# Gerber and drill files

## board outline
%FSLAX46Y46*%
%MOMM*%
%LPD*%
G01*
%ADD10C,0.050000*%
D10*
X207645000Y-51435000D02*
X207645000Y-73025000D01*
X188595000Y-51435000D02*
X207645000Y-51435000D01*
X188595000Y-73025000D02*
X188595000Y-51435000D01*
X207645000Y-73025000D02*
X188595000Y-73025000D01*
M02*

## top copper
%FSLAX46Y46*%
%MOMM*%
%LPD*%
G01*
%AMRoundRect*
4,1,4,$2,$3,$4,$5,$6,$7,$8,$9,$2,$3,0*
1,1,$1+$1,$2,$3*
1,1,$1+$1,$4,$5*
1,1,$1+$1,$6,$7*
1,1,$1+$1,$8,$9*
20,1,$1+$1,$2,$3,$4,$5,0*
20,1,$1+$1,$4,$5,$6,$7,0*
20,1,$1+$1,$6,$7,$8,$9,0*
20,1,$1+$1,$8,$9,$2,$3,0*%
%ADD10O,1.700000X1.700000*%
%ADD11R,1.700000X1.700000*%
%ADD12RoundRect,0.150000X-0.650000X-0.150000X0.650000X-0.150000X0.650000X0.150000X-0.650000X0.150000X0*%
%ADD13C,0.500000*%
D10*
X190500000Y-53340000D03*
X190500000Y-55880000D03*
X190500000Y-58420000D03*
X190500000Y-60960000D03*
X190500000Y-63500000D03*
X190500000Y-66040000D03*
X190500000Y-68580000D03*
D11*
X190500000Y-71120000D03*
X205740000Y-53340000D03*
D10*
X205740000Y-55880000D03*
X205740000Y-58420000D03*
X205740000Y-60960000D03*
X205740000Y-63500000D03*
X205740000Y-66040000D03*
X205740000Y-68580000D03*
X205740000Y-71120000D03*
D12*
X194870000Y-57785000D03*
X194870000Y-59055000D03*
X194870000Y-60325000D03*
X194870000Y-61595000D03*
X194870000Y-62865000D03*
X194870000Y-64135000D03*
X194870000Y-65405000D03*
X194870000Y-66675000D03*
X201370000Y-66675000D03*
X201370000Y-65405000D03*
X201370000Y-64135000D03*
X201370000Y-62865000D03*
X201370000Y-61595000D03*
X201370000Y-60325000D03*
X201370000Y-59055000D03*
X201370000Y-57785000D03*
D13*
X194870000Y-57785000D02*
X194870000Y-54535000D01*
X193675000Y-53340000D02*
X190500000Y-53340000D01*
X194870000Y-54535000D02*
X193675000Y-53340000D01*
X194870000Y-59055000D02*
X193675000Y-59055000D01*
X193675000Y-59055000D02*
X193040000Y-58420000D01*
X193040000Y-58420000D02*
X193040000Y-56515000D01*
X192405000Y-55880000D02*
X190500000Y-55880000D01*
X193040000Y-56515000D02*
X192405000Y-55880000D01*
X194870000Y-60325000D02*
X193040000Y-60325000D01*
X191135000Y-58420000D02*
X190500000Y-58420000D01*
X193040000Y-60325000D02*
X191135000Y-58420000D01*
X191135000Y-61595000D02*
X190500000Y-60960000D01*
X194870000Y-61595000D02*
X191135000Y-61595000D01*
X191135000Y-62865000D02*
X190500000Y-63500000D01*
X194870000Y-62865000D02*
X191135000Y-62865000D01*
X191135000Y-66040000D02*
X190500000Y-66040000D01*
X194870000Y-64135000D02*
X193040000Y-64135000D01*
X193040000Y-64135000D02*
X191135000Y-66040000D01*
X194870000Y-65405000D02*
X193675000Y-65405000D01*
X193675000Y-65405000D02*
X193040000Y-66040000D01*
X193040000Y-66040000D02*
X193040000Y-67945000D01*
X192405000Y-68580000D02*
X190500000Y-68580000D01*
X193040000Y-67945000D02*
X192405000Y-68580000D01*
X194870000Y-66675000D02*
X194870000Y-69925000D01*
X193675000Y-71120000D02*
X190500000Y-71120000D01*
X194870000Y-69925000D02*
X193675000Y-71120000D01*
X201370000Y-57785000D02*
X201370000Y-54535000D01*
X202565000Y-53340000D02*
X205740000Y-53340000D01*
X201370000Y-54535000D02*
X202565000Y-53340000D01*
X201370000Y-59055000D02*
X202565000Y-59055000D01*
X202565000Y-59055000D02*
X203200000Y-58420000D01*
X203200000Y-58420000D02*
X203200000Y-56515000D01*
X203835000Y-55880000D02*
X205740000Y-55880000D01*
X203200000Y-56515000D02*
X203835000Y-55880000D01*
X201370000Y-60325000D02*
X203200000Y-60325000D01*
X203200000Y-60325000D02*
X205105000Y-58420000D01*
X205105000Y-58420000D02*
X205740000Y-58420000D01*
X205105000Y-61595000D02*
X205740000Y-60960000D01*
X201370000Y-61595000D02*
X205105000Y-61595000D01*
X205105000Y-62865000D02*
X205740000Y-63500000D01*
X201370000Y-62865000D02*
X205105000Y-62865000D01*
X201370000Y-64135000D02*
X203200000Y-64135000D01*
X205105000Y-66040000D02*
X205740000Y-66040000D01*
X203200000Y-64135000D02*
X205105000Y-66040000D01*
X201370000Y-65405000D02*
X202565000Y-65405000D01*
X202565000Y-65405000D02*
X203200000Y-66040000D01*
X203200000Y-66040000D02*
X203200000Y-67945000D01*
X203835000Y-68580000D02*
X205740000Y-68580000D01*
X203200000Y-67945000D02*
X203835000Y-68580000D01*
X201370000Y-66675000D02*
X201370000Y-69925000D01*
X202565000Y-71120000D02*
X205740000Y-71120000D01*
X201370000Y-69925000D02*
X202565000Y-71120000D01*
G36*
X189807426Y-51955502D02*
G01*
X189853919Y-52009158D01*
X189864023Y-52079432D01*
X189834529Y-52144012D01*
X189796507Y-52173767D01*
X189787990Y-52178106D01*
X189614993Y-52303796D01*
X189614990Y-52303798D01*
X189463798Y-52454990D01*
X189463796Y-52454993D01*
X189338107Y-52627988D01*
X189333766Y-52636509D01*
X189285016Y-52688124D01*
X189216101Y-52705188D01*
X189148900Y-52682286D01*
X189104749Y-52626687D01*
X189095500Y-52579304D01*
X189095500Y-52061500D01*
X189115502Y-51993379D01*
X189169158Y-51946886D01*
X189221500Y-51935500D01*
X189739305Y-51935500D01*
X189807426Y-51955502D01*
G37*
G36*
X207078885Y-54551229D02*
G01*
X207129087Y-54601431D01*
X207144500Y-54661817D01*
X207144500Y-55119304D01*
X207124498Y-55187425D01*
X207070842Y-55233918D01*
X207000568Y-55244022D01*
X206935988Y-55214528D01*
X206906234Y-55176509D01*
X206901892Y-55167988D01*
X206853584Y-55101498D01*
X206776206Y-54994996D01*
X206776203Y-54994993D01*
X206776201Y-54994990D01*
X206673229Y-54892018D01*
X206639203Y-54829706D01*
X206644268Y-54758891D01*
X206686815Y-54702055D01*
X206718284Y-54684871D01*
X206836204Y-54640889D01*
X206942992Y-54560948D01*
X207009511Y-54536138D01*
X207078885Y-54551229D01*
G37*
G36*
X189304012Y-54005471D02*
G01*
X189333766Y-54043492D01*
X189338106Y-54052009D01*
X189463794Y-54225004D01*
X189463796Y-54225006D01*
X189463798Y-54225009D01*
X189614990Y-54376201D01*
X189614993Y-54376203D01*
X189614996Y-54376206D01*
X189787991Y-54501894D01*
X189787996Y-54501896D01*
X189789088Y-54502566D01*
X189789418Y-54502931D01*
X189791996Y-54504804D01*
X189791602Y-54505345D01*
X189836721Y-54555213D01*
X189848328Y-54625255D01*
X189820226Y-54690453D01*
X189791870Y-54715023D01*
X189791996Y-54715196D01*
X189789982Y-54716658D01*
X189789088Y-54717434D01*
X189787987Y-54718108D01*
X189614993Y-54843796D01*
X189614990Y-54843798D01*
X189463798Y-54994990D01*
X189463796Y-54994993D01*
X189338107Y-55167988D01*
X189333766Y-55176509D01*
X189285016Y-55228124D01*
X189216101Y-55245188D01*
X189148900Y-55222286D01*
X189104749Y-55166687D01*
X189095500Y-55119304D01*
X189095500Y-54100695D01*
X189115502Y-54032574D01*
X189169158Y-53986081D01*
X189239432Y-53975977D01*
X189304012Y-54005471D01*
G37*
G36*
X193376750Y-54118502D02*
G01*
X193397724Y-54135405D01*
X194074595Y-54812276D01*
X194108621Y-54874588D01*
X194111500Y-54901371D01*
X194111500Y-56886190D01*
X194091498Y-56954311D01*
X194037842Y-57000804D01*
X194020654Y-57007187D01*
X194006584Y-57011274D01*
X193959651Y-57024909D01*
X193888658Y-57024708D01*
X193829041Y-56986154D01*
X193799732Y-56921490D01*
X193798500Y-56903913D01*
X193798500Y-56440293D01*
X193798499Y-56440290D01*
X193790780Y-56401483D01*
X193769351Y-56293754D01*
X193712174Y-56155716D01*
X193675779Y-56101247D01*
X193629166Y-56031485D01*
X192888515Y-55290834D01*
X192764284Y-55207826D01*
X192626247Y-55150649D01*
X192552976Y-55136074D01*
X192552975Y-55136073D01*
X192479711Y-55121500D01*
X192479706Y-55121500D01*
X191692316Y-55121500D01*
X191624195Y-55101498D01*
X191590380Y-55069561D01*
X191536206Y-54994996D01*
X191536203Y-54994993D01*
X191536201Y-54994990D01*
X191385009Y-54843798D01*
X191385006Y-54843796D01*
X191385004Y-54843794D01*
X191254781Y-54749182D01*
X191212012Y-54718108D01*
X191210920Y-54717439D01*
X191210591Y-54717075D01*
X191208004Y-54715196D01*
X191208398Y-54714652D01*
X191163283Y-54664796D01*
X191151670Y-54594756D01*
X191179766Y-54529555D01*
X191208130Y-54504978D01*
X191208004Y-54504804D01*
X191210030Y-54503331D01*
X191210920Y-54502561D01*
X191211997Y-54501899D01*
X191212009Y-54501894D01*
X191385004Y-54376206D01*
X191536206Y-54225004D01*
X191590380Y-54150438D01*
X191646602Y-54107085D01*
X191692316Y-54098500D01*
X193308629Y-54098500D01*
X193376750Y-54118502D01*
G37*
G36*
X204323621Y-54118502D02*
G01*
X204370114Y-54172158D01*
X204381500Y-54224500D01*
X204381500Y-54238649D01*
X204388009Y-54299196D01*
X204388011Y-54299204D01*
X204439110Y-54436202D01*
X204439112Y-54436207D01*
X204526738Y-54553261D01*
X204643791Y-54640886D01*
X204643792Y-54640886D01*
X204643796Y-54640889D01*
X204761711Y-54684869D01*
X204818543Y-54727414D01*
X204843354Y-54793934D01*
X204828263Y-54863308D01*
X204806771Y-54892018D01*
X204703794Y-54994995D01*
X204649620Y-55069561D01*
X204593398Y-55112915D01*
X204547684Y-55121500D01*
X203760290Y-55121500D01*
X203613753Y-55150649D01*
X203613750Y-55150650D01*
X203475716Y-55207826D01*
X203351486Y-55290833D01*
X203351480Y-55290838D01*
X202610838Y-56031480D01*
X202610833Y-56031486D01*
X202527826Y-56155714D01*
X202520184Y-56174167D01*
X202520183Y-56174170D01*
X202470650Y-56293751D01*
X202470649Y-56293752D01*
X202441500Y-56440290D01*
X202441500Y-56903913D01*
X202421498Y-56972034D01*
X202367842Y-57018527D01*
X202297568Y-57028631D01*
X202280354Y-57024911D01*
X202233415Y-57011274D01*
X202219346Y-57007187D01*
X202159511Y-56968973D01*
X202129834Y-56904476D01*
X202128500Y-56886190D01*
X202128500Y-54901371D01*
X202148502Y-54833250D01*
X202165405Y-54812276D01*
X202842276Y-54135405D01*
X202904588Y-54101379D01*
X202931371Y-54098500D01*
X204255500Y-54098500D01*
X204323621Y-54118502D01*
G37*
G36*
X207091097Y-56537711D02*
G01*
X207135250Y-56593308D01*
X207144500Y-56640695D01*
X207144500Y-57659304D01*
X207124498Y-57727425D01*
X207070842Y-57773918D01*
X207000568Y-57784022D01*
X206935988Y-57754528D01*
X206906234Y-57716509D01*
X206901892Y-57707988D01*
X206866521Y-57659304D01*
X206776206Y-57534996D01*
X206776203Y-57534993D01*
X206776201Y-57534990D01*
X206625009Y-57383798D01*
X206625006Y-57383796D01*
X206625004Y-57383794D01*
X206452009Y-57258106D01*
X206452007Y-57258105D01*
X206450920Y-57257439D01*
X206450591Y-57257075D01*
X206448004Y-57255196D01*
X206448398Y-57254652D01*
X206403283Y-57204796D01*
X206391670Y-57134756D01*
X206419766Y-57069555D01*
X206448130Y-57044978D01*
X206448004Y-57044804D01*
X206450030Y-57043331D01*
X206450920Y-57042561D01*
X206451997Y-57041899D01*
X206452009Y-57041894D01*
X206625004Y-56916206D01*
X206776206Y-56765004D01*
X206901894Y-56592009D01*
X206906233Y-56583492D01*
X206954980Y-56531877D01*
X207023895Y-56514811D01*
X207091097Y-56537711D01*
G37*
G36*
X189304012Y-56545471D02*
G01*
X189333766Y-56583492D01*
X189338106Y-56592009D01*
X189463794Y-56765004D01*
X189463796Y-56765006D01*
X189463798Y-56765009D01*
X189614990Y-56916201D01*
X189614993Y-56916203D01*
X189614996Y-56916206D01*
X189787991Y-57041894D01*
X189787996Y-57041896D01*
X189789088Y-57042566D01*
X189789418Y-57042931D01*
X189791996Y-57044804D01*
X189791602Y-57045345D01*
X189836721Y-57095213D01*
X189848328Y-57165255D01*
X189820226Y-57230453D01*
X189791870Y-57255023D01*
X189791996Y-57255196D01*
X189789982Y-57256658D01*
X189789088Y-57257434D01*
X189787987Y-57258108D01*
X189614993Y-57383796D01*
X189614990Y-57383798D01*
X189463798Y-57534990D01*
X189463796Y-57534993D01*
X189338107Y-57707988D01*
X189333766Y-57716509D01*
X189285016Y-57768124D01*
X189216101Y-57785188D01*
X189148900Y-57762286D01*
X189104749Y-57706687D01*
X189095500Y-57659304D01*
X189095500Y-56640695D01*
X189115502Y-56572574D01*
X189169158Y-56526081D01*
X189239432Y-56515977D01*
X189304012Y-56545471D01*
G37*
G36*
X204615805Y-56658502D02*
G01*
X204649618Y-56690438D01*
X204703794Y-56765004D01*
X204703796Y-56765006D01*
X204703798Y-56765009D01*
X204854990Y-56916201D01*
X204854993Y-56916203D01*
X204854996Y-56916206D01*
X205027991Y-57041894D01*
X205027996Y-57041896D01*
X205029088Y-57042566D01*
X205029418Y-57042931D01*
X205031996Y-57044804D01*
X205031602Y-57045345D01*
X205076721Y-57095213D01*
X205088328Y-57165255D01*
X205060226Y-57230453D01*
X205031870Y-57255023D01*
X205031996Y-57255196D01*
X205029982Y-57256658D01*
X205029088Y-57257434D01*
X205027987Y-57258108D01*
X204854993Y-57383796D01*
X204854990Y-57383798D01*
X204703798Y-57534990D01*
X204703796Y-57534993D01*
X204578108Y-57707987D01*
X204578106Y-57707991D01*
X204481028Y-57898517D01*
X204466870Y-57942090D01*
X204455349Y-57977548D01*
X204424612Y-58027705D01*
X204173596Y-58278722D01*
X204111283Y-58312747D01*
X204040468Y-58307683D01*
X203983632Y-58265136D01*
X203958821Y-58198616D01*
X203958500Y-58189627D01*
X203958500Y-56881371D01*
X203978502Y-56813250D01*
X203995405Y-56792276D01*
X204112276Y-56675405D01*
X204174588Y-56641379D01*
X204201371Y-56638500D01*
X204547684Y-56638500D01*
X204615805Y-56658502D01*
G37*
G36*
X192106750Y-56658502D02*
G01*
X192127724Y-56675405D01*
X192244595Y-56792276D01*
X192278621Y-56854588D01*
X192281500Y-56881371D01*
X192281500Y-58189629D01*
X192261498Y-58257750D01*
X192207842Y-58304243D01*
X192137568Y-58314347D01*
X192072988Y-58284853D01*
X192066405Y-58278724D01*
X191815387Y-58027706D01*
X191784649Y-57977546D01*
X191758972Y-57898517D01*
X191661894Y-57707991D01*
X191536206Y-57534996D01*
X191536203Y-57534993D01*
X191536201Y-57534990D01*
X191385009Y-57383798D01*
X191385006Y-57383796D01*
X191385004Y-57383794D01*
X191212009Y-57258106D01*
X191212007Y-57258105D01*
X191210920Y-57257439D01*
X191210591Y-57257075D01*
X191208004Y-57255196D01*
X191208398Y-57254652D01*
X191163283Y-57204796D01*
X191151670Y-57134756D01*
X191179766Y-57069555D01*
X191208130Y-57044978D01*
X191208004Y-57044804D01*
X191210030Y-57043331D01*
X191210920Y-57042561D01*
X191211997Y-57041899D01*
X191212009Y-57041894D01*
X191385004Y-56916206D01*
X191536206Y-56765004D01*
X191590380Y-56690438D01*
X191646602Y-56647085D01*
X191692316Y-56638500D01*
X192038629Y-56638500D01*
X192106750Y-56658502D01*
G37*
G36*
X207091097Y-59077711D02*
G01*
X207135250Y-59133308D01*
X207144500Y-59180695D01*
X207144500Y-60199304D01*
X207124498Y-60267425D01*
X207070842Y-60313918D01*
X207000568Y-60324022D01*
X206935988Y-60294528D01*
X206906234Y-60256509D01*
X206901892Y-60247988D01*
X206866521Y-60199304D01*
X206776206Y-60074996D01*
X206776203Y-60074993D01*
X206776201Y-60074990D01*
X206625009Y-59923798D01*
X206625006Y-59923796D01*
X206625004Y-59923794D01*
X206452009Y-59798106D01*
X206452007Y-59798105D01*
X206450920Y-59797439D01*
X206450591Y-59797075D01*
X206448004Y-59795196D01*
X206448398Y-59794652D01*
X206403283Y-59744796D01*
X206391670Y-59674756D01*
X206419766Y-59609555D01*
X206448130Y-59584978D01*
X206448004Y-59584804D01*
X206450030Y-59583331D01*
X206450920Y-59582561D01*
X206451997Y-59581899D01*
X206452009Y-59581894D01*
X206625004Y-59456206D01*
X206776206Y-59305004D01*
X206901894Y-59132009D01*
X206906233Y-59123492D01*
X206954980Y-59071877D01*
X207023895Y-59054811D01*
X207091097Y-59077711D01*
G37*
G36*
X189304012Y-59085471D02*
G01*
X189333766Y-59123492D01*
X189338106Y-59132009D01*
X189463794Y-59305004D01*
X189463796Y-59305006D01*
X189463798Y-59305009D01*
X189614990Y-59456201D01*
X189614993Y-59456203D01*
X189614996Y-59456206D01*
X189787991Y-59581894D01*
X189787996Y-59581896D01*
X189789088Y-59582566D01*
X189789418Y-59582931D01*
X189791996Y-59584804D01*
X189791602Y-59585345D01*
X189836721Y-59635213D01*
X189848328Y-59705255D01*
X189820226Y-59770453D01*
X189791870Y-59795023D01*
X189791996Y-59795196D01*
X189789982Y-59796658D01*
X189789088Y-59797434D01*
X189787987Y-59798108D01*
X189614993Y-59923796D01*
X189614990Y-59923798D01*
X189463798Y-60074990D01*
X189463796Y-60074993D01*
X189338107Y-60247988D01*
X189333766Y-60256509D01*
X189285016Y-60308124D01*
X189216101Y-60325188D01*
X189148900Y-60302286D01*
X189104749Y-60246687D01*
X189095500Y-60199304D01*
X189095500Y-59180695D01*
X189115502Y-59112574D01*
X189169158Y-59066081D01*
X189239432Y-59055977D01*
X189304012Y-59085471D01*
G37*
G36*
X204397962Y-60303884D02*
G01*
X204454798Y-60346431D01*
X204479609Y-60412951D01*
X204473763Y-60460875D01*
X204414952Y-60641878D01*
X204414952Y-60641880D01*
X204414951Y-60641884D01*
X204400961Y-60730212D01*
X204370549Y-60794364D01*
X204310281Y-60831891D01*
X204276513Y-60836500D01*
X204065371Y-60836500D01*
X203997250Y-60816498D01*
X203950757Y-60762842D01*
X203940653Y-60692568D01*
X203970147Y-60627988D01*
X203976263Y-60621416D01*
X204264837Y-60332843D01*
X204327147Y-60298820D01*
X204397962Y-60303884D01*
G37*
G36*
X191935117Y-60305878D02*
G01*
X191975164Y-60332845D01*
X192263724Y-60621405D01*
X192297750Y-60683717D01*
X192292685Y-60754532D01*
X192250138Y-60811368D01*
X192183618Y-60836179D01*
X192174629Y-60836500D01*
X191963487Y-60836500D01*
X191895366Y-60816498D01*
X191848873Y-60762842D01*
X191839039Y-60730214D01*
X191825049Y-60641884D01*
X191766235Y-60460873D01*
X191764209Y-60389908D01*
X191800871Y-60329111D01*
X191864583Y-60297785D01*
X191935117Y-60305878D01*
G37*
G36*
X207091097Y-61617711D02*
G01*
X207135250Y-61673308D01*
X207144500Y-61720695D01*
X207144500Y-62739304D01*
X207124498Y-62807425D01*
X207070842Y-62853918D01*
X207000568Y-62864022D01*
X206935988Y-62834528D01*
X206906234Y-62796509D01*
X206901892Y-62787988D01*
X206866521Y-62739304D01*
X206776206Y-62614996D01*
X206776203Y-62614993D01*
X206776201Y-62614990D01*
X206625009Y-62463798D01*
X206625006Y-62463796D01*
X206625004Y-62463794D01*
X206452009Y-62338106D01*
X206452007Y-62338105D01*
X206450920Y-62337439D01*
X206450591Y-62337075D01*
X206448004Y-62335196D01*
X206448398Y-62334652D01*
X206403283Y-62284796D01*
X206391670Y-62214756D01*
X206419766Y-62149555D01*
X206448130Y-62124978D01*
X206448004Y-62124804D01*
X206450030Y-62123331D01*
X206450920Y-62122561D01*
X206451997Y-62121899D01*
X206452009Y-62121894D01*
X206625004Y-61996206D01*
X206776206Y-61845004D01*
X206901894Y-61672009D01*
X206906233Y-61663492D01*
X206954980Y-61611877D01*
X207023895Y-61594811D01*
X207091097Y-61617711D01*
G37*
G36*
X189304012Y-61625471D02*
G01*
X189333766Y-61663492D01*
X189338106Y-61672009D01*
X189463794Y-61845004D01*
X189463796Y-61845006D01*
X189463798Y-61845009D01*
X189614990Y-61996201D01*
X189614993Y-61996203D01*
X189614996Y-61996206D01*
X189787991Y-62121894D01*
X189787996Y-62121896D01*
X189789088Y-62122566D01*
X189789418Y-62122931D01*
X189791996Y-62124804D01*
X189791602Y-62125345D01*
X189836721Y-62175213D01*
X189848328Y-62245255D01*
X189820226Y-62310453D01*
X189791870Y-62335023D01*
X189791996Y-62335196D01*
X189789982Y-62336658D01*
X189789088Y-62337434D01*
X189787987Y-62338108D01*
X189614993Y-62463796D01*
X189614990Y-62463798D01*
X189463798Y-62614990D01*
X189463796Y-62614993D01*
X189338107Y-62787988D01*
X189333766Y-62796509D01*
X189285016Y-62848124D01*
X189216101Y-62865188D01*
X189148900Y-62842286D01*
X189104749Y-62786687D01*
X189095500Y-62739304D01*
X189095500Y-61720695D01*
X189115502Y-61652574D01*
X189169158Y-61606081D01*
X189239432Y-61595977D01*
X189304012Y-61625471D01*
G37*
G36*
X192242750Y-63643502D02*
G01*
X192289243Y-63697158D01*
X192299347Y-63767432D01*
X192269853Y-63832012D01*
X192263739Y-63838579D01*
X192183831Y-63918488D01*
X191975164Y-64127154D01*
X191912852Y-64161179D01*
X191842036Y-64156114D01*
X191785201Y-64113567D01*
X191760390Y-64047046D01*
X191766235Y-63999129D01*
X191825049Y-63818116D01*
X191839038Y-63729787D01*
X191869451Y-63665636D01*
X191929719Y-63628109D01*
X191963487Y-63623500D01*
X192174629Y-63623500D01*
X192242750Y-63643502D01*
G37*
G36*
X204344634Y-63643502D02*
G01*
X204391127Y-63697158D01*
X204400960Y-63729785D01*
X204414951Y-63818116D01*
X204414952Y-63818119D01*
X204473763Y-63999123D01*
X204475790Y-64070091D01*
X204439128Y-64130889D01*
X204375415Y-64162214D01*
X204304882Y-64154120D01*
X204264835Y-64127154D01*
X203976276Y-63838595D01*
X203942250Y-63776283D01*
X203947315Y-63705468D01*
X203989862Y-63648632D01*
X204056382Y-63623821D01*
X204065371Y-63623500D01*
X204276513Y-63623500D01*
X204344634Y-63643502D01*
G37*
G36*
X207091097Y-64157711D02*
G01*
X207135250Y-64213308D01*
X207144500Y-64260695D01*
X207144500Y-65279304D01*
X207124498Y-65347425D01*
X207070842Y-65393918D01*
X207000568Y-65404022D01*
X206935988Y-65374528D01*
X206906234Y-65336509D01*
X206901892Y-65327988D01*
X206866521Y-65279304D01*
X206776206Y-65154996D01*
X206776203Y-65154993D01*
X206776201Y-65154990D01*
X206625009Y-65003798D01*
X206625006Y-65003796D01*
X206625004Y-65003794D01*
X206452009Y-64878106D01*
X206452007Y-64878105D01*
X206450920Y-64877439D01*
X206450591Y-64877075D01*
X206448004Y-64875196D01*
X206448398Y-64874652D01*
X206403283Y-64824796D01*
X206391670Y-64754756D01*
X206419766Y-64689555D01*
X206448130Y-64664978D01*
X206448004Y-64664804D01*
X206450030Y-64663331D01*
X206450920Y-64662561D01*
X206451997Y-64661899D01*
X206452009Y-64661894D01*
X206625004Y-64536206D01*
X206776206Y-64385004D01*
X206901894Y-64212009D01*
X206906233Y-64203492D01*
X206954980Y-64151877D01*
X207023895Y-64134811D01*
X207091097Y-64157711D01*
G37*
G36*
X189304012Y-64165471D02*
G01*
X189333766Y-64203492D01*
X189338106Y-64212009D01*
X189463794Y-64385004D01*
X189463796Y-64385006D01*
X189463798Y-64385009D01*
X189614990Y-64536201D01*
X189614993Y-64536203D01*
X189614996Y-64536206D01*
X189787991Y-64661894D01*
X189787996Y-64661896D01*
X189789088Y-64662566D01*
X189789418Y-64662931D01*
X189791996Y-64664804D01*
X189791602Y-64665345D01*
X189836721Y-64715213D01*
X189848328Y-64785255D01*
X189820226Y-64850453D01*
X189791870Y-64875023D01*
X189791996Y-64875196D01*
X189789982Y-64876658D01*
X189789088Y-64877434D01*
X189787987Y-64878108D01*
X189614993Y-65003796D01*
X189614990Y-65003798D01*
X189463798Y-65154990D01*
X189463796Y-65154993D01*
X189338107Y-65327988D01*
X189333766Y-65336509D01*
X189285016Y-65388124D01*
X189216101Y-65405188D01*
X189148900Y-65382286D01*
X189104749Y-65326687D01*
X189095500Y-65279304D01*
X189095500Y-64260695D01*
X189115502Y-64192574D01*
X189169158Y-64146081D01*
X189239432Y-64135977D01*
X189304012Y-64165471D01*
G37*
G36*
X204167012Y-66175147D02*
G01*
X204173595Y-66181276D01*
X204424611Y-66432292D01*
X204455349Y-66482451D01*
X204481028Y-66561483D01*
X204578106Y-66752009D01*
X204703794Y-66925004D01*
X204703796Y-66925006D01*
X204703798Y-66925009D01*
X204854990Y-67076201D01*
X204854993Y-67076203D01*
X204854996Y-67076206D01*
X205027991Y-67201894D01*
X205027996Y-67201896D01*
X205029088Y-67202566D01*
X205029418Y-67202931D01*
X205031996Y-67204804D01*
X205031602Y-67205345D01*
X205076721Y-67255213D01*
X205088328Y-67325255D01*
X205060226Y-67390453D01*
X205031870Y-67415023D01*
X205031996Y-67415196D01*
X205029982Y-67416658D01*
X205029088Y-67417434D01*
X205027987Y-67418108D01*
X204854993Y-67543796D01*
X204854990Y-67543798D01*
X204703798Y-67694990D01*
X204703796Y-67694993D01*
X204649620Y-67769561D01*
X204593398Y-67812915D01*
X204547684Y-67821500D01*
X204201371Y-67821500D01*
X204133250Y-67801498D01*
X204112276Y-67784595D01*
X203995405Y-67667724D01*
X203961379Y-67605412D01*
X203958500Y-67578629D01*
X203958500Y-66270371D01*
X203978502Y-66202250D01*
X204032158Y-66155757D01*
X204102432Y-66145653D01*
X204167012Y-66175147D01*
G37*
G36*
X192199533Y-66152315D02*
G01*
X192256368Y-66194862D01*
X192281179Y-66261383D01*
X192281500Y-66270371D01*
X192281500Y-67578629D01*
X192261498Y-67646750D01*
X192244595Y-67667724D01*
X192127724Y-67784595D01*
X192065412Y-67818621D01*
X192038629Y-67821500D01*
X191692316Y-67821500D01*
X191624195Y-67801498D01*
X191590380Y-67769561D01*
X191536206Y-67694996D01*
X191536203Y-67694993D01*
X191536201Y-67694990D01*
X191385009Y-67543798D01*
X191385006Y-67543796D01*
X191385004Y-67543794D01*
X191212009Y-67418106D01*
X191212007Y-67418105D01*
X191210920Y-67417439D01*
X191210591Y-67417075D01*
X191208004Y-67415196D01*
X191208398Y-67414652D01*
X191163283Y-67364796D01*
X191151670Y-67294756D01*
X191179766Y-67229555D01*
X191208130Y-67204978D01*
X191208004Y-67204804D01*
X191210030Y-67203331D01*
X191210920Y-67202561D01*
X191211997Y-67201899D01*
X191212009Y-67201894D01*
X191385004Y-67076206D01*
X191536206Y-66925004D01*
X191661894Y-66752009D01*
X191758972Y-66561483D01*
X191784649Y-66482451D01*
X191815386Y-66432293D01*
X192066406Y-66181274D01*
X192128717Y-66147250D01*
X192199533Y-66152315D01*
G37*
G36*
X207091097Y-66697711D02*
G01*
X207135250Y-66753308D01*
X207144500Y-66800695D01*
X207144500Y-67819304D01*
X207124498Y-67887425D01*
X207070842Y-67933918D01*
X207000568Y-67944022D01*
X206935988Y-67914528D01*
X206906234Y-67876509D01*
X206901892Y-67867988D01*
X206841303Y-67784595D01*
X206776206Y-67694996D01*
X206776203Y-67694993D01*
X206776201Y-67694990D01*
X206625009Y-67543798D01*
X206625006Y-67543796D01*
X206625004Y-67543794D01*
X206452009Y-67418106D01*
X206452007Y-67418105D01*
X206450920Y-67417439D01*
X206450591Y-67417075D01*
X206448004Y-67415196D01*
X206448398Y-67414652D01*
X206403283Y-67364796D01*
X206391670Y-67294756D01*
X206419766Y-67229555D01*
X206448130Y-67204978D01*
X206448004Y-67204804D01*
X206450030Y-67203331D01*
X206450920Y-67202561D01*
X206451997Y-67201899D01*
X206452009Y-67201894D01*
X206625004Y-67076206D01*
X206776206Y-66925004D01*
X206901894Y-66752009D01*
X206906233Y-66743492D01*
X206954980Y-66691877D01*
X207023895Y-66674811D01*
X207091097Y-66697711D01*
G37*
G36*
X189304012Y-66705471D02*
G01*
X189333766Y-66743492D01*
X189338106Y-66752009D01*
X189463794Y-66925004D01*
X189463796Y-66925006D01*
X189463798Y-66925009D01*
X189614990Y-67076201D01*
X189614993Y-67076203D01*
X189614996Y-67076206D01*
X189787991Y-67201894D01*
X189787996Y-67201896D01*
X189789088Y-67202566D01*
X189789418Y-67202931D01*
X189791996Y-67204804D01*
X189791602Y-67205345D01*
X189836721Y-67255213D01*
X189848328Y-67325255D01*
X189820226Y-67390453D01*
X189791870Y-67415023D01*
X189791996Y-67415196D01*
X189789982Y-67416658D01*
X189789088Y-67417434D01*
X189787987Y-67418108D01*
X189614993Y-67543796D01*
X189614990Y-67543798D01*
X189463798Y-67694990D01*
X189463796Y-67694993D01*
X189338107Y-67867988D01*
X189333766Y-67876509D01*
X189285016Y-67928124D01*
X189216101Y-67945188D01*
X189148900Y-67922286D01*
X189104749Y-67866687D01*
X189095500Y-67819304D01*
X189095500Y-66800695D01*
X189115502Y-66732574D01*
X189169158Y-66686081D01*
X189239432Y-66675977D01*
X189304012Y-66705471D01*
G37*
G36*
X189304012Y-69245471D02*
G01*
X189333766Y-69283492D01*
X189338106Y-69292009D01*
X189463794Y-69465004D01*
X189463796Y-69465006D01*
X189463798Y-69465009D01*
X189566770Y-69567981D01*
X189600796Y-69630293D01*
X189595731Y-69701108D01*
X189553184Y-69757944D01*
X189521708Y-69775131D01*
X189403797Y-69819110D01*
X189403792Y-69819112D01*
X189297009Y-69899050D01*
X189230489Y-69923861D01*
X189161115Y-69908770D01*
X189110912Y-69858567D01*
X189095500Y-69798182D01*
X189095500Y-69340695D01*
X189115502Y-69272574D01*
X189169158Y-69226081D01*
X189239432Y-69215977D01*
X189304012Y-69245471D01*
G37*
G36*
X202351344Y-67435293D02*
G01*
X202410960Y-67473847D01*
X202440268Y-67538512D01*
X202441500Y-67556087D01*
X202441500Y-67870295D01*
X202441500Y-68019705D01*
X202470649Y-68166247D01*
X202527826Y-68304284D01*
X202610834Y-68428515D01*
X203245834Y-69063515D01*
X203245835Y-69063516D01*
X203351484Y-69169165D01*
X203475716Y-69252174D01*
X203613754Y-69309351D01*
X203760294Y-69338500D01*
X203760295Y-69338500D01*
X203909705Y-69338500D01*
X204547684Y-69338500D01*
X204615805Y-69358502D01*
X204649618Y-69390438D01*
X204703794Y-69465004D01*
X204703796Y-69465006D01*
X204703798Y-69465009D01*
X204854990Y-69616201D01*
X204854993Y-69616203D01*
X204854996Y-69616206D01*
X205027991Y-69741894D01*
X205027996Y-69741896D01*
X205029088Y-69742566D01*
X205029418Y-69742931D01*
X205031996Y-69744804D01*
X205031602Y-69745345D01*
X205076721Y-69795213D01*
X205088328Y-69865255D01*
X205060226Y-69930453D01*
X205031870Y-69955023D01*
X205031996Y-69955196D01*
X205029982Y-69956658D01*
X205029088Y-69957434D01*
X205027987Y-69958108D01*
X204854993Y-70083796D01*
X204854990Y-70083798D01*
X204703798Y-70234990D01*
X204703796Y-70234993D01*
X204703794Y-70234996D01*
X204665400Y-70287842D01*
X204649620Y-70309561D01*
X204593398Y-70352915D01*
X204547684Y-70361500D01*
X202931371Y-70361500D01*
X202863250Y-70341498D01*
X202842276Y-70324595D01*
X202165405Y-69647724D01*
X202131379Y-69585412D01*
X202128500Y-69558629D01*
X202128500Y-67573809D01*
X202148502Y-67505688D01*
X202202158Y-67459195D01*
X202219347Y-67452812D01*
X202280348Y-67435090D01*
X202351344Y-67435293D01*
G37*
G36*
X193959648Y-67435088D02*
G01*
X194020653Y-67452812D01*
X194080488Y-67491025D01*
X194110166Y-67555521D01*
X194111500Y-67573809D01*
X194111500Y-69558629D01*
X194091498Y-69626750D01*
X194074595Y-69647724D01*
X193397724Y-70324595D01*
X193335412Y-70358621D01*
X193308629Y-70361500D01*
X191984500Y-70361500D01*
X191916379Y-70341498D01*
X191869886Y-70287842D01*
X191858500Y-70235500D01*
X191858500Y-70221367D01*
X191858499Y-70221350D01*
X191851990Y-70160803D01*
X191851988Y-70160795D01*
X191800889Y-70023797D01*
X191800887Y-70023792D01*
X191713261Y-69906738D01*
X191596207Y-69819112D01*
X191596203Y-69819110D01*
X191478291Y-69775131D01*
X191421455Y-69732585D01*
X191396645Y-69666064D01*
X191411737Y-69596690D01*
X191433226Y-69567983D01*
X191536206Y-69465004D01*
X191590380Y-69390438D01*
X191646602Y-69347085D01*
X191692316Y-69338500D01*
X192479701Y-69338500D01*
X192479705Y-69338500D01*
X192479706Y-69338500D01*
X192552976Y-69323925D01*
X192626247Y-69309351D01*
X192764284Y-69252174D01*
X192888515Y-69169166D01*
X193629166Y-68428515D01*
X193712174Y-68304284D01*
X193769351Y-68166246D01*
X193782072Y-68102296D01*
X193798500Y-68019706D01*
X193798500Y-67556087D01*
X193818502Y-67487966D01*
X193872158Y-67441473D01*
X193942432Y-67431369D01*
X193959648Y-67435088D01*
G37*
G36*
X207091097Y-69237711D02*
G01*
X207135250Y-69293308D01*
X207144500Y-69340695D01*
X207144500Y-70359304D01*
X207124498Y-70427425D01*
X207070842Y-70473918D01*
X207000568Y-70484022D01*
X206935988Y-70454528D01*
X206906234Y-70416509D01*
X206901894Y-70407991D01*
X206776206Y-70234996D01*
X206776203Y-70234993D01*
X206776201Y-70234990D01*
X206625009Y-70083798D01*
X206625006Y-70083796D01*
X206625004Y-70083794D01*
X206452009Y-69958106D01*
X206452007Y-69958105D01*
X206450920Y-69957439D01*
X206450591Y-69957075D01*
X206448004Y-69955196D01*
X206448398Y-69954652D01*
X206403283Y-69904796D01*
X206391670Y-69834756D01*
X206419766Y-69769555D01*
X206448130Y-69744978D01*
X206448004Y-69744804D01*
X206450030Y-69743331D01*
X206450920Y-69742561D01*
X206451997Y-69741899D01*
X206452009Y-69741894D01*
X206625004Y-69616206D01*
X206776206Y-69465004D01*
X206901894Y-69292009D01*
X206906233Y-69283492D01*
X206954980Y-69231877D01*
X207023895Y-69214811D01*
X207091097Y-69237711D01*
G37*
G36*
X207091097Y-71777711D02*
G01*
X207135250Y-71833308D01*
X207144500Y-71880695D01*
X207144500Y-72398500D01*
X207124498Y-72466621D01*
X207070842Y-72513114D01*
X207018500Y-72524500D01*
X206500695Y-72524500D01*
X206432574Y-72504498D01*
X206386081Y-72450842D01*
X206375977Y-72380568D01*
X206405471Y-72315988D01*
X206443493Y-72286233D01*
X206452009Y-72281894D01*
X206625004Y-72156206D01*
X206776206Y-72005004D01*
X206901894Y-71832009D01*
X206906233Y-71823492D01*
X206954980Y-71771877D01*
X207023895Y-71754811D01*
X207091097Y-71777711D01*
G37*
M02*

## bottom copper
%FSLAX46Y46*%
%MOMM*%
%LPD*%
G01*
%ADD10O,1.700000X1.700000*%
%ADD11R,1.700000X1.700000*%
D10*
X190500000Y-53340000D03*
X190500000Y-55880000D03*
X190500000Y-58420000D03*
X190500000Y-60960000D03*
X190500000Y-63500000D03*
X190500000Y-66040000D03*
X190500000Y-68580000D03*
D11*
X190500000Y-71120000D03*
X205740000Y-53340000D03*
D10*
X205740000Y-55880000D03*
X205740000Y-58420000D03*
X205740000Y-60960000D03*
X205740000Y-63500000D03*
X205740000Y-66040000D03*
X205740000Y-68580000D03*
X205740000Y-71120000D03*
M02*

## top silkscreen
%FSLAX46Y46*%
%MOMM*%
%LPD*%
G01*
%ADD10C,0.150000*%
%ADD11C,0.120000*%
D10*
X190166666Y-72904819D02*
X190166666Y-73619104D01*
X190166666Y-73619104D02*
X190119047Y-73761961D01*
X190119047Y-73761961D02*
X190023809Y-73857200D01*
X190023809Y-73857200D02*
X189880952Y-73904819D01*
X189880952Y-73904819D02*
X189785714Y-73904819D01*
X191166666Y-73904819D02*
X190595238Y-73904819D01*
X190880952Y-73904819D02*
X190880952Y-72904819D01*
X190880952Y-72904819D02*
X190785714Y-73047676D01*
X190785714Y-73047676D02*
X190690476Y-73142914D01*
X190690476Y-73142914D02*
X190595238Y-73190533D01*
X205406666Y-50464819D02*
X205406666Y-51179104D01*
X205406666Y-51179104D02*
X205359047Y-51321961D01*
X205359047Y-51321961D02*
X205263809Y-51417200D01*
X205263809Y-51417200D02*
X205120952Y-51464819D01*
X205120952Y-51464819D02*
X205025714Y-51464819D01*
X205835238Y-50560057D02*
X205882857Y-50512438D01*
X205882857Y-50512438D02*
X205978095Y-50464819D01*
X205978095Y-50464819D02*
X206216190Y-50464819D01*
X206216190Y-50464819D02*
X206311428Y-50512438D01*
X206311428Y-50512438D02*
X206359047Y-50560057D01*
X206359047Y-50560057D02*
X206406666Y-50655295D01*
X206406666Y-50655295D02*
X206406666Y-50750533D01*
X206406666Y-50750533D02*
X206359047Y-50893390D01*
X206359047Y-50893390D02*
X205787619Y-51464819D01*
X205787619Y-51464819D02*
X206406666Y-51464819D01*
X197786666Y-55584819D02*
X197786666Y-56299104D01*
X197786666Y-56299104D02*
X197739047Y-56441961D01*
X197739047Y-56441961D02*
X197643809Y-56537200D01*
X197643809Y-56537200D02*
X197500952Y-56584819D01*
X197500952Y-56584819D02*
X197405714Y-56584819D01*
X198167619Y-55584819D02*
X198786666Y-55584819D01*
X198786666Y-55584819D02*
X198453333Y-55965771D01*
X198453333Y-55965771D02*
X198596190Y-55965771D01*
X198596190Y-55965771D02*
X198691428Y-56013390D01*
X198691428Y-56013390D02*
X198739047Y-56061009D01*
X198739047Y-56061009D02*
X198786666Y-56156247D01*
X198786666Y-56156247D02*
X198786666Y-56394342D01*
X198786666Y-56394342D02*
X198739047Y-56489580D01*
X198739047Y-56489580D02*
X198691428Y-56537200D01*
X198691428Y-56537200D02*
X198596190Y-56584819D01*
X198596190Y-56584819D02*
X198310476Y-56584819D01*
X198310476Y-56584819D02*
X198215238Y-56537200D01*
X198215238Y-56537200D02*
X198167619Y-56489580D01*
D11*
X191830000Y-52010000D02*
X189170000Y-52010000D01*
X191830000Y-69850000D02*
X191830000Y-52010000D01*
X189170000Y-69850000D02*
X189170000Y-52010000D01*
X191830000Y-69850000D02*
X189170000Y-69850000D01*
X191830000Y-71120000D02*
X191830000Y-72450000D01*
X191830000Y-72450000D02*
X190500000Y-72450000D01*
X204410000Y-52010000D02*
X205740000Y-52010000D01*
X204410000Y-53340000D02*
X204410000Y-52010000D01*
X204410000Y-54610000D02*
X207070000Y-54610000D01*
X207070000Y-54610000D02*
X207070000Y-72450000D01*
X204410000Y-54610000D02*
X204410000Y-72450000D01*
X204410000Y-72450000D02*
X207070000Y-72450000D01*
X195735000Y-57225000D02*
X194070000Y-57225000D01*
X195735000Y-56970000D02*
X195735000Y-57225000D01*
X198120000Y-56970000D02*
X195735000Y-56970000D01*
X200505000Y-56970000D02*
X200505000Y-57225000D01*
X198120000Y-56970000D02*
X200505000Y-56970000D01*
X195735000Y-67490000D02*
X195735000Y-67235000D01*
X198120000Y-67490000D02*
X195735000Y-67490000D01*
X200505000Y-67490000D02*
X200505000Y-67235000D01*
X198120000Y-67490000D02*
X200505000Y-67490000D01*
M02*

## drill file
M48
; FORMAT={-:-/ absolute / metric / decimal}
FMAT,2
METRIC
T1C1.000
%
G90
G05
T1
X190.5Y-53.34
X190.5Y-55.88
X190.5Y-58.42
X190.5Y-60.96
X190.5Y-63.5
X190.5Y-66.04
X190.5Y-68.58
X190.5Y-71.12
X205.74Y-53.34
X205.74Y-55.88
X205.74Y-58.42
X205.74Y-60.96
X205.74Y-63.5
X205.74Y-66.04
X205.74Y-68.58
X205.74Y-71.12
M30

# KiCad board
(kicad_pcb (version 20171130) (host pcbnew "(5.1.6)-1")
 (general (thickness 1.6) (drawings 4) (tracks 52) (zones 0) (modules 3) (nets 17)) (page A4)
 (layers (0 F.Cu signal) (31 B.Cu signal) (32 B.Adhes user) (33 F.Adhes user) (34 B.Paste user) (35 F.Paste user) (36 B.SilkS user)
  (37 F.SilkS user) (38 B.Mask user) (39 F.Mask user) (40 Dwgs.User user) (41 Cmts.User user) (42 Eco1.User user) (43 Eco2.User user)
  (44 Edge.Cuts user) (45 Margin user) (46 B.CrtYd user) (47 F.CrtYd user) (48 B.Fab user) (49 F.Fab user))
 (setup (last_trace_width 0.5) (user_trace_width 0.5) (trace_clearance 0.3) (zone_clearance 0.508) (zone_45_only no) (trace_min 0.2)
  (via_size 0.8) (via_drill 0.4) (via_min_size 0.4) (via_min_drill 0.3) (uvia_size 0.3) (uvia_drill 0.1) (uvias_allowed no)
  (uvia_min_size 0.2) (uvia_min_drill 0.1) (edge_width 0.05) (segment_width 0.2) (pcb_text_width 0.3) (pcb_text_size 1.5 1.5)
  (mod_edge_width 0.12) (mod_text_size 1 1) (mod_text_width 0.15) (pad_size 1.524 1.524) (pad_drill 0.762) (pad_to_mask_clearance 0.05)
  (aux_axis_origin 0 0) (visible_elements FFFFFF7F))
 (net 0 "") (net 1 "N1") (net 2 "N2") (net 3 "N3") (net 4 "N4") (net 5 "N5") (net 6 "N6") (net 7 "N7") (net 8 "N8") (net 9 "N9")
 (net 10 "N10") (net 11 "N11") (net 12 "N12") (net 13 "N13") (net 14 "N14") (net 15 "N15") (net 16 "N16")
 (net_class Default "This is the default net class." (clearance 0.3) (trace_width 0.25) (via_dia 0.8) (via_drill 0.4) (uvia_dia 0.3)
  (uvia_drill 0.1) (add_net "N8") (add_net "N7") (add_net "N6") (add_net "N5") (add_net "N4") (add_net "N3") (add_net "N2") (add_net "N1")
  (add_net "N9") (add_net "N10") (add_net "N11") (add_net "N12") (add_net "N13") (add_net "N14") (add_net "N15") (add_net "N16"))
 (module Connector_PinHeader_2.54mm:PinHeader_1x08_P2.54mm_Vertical (layer F.Cu) (at 190.5 71.12 180)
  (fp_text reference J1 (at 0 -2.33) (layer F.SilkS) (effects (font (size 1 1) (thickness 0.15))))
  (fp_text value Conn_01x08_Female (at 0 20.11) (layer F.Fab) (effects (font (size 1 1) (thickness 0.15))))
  (fp_line (start -1.33 19.11) (end 1.33 19.11) (layer F.SilkS) (width 0.12))
  (fp_line (start -1.33 1.27) (end -1.33 19.11) (layer F.SilkS) (width 0.12))
  (fp_line (start 1.33 1.27) (end 1.33 19.11) (layer F.SilkS) (width 0.12))
  (fp_line (start -1.33 1.27) (end 1.33 1.27) (layer F.SilkS) (width 0.12))
  (fp_line (start -1.33 0) (end -1.33 -1.33) (layer F.SilkS) (width 0.12))
  (fp_line (start -1.33 -1.33) (end 0 -1.33) (layer F.SilkS) (width 0.12))
  (pad 8 thru_hole oval (at 0 17.78 180) (size 1.7 1.7) (drill 1) (layers *.Cu *.Mask) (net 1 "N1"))
  (pad 7 thru_hole oval (at 0 15.24 180) (size 1.7 1.7) (drill 1) (layers *.Cu *.Mask) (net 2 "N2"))
  (pad 6 thru_hole oval (at 0 12.7 180) (size 1.7 1.7) (drill 1) (layers *.Cu *.Mask) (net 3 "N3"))
  (pad 5 thru_hole oval (at 0 10.16 180) (size 1.7 1.7) (drill 1) (layers *.Cu *.Mask) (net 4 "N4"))
  (pad 4 thru_hole oval (at 0 7.62 180) (size 1.7 1.7) (drill 1) (layers *.Cu *.Mask) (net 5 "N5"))
  (pad 3 thru_hole oval (at 0 5.08 180) (size 1.7 1.7) (drill 1) (layers *.Cu *.Mask) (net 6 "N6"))
  (pad 2 thru_hole oval (at 0 2.54 180) (size 1.7 1.7) (drill 1) (layers *.Cu *.Mask) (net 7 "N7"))
  (pad 1 thru_hole rect (at 0 0 180) (size 1.7 1.7) (drill 1) (layers *.Cu *.Mask) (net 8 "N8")))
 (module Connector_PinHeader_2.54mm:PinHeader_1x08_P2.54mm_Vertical (layer F.Cu) (at 205.74 53.34)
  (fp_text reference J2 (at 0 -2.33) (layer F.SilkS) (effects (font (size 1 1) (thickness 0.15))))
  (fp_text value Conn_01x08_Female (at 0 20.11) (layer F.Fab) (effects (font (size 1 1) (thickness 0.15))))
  (fp_line (start -1.33 -1.33) (end 0 -1.33) (layer F.SilkS) (width 0.12))
  (fp_line (start -1.33 0) (end -1.33 -1.33) (layer F.SilkS) (width 0.12))
  (fp_line (start -1.33 1.27) (end 1.33 1.27) (layer F.SilkS) (width 0.12))
  (fp_line (start 1.33 1.27) (end 1.33 19.11) (layer F.SilkS) (width 0.12))
  (fp_line (start -1.33 1.27) (end -1.33 19.11) (layer F.SilkS) (width 0.12))
  (fp_line (start -1.33 19.11) (end 1.33 19.11) (layer F.SilkS) (width 0.12))
  (pad 1 thru_hole rect (at 0 0) (size 1.7 1.7) (drill 1) (layers *.Cu *.Mask) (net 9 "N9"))
  (pad 2 thru_hole oval (at 0 2.54) (size 1.7 1.7) (drill 1) (layers *.Cu *.Mask) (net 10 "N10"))
  (pad 3 thru_hole oval (at 0 5.08) (size 1.7 1.7) (drill 1) (layers *.Cu *.Mask) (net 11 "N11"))
  (pad 4 thru_hole oval (at 0 7.62) (size 1.7 1.7) (drill 1) (layers *.Cu *.Mask) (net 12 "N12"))
  (pad 5 thru_hole oval (at 0 10.16) (size 1.7 1.7) (drill 1) (layers *.Cu *.Mask) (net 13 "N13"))
  (pad 6 thru_hole oval (at 0 12.7) (size 1.7 1.7) (drill 1) (layers *.Cu *.Mask) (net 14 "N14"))
  (pad 7 thru_hole oval (at 0 15.24) (size 1.7 1.7) (drill 1) (layers *.Cu *.Mask) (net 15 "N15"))
  (pad 8 thru_hole oval (at 0 17.78) (size 1.7 1.7) (drill 1) (layers *.Cu *.Mask) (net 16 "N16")))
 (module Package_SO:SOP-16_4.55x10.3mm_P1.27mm (layer F.Cu) (at 198.12 62.23)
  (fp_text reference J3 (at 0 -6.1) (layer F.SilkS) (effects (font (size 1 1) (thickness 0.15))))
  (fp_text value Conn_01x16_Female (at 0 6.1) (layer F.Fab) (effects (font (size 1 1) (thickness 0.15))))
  (fp_line (start -2.385 -5.005) (end -4.05 -5.005) (layer F.SilkS) (width 0.12))
  (fp_line (start -2.385 -5.26) (end -2.385 -5.005) (layer F.SilkS) (width 0.12))
  (fp_line (start 0 -5.26) (end -2.385 -5.26) (layer F.SilkS) (width 0.12))
  (fp_line (start 2.385 -5.26) (end 2.385 -5.005) (layer F.SilkS) (width 0.12))
  (fp_line (start 0 -5.26) (end 2.385 -5.26) (layer F.SilkS) (width 0.12))
  (fp_line (start -2.385 5.26) (end -2.385 5.005) (layer F.SilkS) (width 0.12))
  (fp_line (start 0 5.26) (end -2.385 5.26) (layer F.SilkS) (width 0.12))
  (fp_line (start 2.385 5.26) (end 2.385 5.005) (layer F.SilkS) (width 0.12))
  (fp_line (start 0 5.26) (end 2.385 5.26) (layer F.SilkS) (width 0.12))
  (pad 1 smd roundrect (at -3.25 -4.445) (size 1.6 0.6) (layers F.Cu F.Paste F.Mask) (roundrect_rratio 0.25) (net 1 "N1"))
  (pad 2 smd roundrect (at -3.25 -3.175) (size 1.6 0.6) (layers F.Cu F.Paste F.Mask) (roundrect_rratio 0.25) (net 2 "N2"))
  (pad 3 smd roundrect (at -3.25 -1.905) (size 1.6 0.6) (layers F.Cu F.Paste F.Mask) (roundrect_rratio 0.25) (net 3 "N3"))
  (pad 4 smd roundrect (at -3.25 -0.635) (size 1.6 0.6) (layers F.Cu F.Paste F.Mask) (roundrect_rratio 0.25) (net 4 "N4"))
  (pad 5 smd roundrect (at -3.25 0.635) (size 1.6 0.6) (layers F.Cu F.Paste F.Mask) (roundrect_rratio 0.25) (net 5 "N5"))
  (pad 6 smd roundrect (at -3.25 1.905) (size 1.6 0.6) (layers F.Cu F.Paste F.Mask) (roundrect_rratio 0.25) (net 6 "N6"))
  (pad 7 smd roundrect (at -3.25 3.175) (size 1.6 0.6) (layers F.Cu F.Paste F.Mask) (roundrect_rratio 0.25) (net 7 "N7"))
  (pad 8 smd roundrect (at -3.25 4.445) (size 1.6 0.6) (layers F.Cu F.Paste F.Mask) (roundrect_rratio 0.25) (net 8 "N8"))
  (pad 9 smd roundrect (at 3.25 4.445) (size 1.6 0.6) (layers F.Cu F.Paste F.Mask) (roundrect_rratio 0.25) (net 16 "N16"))
  (pad 10 smd roundrect (at 3.25 3.175) (size 1.6 0.6) (layers F.Cu F.Paste F.Mask) (roundrect_rratio 0.25) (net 15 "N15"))
  (pad 11 smd roundrect (at 3.25 1.905) (size 1.6 0.6) (layers F.Cu F.Paste F.Mask) (roundrect_rratio 0.25) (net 14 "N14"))
  (pad 12 smd roundrect (at 3.25 0.635) (size 1.6 0.6) (layers F.Cu F.Paste F.Mask) (roundrect_rratio 0.25) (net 13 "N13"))
  (pad 13 smd roundrect (at 3.25 -0.635) (size 1.6 0.6) (layers F.Cu F.Paste F.Mask) (roundrect_rratio 0.25) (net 12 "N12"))
  (pad 14 smd roundrect (at 3.25 -1.905) (size 1.6 0.6) (layers F.Cu F.Paste F.Mask) (roundrect_rratio 0.25) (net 11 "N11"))
  (pad 15 smd roundrect (at 3.25 -3.175) (size 1.6 0.6) (layers F.Cu F.Paste F.Mask) (roundrect_rratio 0.25) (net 10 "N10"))
  (pad 16 smd roundrect (at 3.25 -4.445) (size 1.6 0.6) (layers F.Cu F.Paste F.Mask) (roundrect_rratio 0.25) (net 9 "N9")))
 (gr_line (start 207.645 51.435) (end 207.645 73.025) (layer Edge.Cuts) (width 0.05))
 (gr_line (start 188.595 51.435) (end 207.645 51.435) (layer Edge.Cuts) (width 0.05))
 (gr_line (start 188.595 73.025) (end 188.595 51.435) (layer Edge.Cuts) (width 0.05))
 (gr_line (start 207.645 73.025) (end 188.595 73.025) (layer Edge.Cuts) (width 0.05))
 (segment (start 194.87 57.785) (end 194.87 54.535) (width 0.5) (layer F.Cu) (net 1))
 (segment (start 193.675 53.34) (end 190.5 53.34) (width 0.5) (layer F.Cu) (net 1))
 (segment (start 194.87 54.535) (end 193.675 53.34) (width 0.5) (layer F.Cu) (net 1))
 (segment (start 194.87 59.055) (end 193.675 59.055) (width 0.5) (layer F.Cu) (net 2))
 (segment (start 193.675 59.055) (end 193.04 58.42) (width 0.5) (layer F.Cu) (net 2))
 (segment (start 193.04 58.42) (end 193.04 56.515) (width 0.5) (layer F.Cu) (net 2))
 (segment (start 192.405 55.88) (end 190.5 55.88) (width 0.5) (layer F.Cu) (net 2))
 (segment (start 193.04 56.515) (end 192.405 55.88) (width 0.5) (layer F.Cu) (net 2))
 (segment (start 194.87 60.325) (end 193.04 60.325) (width 0.5) (layer F.Cu) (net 3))
 (segment (start 191.135 58.42) (end 190.5 58.42) (width 0.5) (layer F.Cu) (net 3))
 (segment (start 193.04 60.325) (end 191.135 58.42) (width 0.5) (layer F.Cu) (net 3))
 (segment (start 191.135 61.595) (end 190.5 60.96) (width 0.5) (layer F.Cu) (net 4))
 (segment (start 194.87 61.595) (end 191.135 61.595) (width 0.5) (layer F.Cu) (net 4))
 (segment (start 191.135 62.865) (end 190.5 63.5) (width 0.5) (layer F.Cu) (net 5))
 (segment (start 194.87 62.865) (end 191.135 62.865) (width 0.5) (layer F.Cu) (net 5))
 (segment (start 191.135 66.04) (end 190.5 66.04) (width 0.5) (layer F.Cu) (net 6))
 (segment (start 194.87 64.135) (end 193.04 64.135) (width 0.5) (layer F.Cu) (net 6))
 (segment (start 193.04 64.135) (end 191.135 66.04) (width 0.5) (layer F.Cu) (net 6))
 (segment (start 194.87 65.405) (end 193.675 65.405) (width 0.5) (layer F.Cu) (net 7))
 (segment (start 193.675 65.405) (end 193.04 66.04) (width 0.5) (layer F.Cu) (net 7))
 (segment (start 193.04 66.04) (end 193.04 67.945) (width 0.5) (layer F.Cu) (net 7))
 (segment (start 192.405 68.58) (end 190.5 68.58) (width 0.5) (layer F.Cu) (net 7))
 (segment (start 193.04 67.945) (end 192.405 68.58) (width 0.5) (layer F.Cu) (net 7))
 (segment (start 194.87 66.675) (end 194.87 69.925) (width 0.5) (layer F.Cu) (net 8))
 (segment (start 193.675 71.12) (end 190.5 71.12) (width 0.5) (layer F.Cu) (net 8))
 (segment (start 194.87 69.925) (end 193.675 71.12) (width 0.5) (layer F.Cu) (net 8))
 (segment (start 201.37 57.785) (end 201.37 54.535) (width 0.5) (layer F.Cu) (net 9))
 (segment (start 202.565 53.34) (end 205.74 53.34) (width 0.5) (layer F.Cu) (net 9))
 (segment (start 201.37 54.535) (end 202.565 53.34) (width 0.5) (layer F.Cu) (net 9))
 (segment (start 201.37 59.055) (end 202.565 59.055) (width 0.5) (layer F.Cu) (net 10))
 (segment (start 202.565 59.055) (end 203.2 58.42) (width 0.5) (layer F.Cu) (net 10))
 (segment (start 203.2 58.42) (end 203.2 56.515) (width 0.5) (layer F.Cu) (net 10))
 (segment (start 203.835 55.88) (end 205.74 55.88) (width 0.5) (layer F.Cu) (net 10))
 (segment (start 203.2 56.515) (end 203.835 55.88) (width 0.5) (layer F.Cu) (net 10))
 (segment (start 201.37 60.325) (end 203.2 60.325) (width 0.5) (layer F.Cu) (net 11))
 (segment (start 203.2 60.325) (end 205.105 58.42) (width 0.5) (layer F.Cu) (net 11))
 (segment (start 205.105 58.42) (end 205.74 58.42) (width 0.5) (layer F.Cu) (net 11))
 (segment (start 205.105 61.595) (end 205.74 60.96) (width 0.5) (layer F.Cu) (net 12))
 (segment (start 201.37 61.595) (end 205.105 61.595) (width 0.5) (layer F.Cu) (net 12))
 (segment (start 205.105 62.865) (end 205.74 63.5) (width 0.5) (layer F.Cu) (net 13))
 (segment (start 201.37 62.865) (end 205.105 62.865) (width 0.5) (layer F.Cu) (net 13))
 (segment (start 201.37 64.135) (end 203.2 64.135) (width 0.5) (layer F.Cu) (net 14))
 (segment (start 205.105 66.04) (end 205.74 66.04) (width 0.5) (layer F.Cu) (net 14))
 (segment (start 203.2 64.135) (end 205.105 66.04) (width 0.5) (layer F.Cu) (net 14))
 (segment (start 201.37 65.405) (end 202.565 65.405) (width 0.5) (layer F.Cu) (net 15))
 (segment (start 202.565 65.405) (end 203.2 66.04) (width 0.5) (layer F.Cu) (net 15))
 (segment (start 203.2 66.04) (end 203.2 67.945) (width 0.5) (layer F.Cu) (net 15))
 (segment (start 203.835 68.58) (end 205.74 68.58) (width 0.5) (layer F.Cu) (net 15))
 (segment (start 203.2 67.945) (end 203.835 68.58) (width 0.5) (layer F.Cu) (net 15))
 (segment (start 201.37 66.675) (end 201.37 69.925) (width 0.5) (layer F.Cu) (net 16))
 (segment (start 202.565 71.12) (end 205.74 71.12) (width 0.5) (layer F.Cu) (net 16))
 (segment (start 201.37 69.925) (end 202.565 71.12) (width 0.5) (layer F.Cu) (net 16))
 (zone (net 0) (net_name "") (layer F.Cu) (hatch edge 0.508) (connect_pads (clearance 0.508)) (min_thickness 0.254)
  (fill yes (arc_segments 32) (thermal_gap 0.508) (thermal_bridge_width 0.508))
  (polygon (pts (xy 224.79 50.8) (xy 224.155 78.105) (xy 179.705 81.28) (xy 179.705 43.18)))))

